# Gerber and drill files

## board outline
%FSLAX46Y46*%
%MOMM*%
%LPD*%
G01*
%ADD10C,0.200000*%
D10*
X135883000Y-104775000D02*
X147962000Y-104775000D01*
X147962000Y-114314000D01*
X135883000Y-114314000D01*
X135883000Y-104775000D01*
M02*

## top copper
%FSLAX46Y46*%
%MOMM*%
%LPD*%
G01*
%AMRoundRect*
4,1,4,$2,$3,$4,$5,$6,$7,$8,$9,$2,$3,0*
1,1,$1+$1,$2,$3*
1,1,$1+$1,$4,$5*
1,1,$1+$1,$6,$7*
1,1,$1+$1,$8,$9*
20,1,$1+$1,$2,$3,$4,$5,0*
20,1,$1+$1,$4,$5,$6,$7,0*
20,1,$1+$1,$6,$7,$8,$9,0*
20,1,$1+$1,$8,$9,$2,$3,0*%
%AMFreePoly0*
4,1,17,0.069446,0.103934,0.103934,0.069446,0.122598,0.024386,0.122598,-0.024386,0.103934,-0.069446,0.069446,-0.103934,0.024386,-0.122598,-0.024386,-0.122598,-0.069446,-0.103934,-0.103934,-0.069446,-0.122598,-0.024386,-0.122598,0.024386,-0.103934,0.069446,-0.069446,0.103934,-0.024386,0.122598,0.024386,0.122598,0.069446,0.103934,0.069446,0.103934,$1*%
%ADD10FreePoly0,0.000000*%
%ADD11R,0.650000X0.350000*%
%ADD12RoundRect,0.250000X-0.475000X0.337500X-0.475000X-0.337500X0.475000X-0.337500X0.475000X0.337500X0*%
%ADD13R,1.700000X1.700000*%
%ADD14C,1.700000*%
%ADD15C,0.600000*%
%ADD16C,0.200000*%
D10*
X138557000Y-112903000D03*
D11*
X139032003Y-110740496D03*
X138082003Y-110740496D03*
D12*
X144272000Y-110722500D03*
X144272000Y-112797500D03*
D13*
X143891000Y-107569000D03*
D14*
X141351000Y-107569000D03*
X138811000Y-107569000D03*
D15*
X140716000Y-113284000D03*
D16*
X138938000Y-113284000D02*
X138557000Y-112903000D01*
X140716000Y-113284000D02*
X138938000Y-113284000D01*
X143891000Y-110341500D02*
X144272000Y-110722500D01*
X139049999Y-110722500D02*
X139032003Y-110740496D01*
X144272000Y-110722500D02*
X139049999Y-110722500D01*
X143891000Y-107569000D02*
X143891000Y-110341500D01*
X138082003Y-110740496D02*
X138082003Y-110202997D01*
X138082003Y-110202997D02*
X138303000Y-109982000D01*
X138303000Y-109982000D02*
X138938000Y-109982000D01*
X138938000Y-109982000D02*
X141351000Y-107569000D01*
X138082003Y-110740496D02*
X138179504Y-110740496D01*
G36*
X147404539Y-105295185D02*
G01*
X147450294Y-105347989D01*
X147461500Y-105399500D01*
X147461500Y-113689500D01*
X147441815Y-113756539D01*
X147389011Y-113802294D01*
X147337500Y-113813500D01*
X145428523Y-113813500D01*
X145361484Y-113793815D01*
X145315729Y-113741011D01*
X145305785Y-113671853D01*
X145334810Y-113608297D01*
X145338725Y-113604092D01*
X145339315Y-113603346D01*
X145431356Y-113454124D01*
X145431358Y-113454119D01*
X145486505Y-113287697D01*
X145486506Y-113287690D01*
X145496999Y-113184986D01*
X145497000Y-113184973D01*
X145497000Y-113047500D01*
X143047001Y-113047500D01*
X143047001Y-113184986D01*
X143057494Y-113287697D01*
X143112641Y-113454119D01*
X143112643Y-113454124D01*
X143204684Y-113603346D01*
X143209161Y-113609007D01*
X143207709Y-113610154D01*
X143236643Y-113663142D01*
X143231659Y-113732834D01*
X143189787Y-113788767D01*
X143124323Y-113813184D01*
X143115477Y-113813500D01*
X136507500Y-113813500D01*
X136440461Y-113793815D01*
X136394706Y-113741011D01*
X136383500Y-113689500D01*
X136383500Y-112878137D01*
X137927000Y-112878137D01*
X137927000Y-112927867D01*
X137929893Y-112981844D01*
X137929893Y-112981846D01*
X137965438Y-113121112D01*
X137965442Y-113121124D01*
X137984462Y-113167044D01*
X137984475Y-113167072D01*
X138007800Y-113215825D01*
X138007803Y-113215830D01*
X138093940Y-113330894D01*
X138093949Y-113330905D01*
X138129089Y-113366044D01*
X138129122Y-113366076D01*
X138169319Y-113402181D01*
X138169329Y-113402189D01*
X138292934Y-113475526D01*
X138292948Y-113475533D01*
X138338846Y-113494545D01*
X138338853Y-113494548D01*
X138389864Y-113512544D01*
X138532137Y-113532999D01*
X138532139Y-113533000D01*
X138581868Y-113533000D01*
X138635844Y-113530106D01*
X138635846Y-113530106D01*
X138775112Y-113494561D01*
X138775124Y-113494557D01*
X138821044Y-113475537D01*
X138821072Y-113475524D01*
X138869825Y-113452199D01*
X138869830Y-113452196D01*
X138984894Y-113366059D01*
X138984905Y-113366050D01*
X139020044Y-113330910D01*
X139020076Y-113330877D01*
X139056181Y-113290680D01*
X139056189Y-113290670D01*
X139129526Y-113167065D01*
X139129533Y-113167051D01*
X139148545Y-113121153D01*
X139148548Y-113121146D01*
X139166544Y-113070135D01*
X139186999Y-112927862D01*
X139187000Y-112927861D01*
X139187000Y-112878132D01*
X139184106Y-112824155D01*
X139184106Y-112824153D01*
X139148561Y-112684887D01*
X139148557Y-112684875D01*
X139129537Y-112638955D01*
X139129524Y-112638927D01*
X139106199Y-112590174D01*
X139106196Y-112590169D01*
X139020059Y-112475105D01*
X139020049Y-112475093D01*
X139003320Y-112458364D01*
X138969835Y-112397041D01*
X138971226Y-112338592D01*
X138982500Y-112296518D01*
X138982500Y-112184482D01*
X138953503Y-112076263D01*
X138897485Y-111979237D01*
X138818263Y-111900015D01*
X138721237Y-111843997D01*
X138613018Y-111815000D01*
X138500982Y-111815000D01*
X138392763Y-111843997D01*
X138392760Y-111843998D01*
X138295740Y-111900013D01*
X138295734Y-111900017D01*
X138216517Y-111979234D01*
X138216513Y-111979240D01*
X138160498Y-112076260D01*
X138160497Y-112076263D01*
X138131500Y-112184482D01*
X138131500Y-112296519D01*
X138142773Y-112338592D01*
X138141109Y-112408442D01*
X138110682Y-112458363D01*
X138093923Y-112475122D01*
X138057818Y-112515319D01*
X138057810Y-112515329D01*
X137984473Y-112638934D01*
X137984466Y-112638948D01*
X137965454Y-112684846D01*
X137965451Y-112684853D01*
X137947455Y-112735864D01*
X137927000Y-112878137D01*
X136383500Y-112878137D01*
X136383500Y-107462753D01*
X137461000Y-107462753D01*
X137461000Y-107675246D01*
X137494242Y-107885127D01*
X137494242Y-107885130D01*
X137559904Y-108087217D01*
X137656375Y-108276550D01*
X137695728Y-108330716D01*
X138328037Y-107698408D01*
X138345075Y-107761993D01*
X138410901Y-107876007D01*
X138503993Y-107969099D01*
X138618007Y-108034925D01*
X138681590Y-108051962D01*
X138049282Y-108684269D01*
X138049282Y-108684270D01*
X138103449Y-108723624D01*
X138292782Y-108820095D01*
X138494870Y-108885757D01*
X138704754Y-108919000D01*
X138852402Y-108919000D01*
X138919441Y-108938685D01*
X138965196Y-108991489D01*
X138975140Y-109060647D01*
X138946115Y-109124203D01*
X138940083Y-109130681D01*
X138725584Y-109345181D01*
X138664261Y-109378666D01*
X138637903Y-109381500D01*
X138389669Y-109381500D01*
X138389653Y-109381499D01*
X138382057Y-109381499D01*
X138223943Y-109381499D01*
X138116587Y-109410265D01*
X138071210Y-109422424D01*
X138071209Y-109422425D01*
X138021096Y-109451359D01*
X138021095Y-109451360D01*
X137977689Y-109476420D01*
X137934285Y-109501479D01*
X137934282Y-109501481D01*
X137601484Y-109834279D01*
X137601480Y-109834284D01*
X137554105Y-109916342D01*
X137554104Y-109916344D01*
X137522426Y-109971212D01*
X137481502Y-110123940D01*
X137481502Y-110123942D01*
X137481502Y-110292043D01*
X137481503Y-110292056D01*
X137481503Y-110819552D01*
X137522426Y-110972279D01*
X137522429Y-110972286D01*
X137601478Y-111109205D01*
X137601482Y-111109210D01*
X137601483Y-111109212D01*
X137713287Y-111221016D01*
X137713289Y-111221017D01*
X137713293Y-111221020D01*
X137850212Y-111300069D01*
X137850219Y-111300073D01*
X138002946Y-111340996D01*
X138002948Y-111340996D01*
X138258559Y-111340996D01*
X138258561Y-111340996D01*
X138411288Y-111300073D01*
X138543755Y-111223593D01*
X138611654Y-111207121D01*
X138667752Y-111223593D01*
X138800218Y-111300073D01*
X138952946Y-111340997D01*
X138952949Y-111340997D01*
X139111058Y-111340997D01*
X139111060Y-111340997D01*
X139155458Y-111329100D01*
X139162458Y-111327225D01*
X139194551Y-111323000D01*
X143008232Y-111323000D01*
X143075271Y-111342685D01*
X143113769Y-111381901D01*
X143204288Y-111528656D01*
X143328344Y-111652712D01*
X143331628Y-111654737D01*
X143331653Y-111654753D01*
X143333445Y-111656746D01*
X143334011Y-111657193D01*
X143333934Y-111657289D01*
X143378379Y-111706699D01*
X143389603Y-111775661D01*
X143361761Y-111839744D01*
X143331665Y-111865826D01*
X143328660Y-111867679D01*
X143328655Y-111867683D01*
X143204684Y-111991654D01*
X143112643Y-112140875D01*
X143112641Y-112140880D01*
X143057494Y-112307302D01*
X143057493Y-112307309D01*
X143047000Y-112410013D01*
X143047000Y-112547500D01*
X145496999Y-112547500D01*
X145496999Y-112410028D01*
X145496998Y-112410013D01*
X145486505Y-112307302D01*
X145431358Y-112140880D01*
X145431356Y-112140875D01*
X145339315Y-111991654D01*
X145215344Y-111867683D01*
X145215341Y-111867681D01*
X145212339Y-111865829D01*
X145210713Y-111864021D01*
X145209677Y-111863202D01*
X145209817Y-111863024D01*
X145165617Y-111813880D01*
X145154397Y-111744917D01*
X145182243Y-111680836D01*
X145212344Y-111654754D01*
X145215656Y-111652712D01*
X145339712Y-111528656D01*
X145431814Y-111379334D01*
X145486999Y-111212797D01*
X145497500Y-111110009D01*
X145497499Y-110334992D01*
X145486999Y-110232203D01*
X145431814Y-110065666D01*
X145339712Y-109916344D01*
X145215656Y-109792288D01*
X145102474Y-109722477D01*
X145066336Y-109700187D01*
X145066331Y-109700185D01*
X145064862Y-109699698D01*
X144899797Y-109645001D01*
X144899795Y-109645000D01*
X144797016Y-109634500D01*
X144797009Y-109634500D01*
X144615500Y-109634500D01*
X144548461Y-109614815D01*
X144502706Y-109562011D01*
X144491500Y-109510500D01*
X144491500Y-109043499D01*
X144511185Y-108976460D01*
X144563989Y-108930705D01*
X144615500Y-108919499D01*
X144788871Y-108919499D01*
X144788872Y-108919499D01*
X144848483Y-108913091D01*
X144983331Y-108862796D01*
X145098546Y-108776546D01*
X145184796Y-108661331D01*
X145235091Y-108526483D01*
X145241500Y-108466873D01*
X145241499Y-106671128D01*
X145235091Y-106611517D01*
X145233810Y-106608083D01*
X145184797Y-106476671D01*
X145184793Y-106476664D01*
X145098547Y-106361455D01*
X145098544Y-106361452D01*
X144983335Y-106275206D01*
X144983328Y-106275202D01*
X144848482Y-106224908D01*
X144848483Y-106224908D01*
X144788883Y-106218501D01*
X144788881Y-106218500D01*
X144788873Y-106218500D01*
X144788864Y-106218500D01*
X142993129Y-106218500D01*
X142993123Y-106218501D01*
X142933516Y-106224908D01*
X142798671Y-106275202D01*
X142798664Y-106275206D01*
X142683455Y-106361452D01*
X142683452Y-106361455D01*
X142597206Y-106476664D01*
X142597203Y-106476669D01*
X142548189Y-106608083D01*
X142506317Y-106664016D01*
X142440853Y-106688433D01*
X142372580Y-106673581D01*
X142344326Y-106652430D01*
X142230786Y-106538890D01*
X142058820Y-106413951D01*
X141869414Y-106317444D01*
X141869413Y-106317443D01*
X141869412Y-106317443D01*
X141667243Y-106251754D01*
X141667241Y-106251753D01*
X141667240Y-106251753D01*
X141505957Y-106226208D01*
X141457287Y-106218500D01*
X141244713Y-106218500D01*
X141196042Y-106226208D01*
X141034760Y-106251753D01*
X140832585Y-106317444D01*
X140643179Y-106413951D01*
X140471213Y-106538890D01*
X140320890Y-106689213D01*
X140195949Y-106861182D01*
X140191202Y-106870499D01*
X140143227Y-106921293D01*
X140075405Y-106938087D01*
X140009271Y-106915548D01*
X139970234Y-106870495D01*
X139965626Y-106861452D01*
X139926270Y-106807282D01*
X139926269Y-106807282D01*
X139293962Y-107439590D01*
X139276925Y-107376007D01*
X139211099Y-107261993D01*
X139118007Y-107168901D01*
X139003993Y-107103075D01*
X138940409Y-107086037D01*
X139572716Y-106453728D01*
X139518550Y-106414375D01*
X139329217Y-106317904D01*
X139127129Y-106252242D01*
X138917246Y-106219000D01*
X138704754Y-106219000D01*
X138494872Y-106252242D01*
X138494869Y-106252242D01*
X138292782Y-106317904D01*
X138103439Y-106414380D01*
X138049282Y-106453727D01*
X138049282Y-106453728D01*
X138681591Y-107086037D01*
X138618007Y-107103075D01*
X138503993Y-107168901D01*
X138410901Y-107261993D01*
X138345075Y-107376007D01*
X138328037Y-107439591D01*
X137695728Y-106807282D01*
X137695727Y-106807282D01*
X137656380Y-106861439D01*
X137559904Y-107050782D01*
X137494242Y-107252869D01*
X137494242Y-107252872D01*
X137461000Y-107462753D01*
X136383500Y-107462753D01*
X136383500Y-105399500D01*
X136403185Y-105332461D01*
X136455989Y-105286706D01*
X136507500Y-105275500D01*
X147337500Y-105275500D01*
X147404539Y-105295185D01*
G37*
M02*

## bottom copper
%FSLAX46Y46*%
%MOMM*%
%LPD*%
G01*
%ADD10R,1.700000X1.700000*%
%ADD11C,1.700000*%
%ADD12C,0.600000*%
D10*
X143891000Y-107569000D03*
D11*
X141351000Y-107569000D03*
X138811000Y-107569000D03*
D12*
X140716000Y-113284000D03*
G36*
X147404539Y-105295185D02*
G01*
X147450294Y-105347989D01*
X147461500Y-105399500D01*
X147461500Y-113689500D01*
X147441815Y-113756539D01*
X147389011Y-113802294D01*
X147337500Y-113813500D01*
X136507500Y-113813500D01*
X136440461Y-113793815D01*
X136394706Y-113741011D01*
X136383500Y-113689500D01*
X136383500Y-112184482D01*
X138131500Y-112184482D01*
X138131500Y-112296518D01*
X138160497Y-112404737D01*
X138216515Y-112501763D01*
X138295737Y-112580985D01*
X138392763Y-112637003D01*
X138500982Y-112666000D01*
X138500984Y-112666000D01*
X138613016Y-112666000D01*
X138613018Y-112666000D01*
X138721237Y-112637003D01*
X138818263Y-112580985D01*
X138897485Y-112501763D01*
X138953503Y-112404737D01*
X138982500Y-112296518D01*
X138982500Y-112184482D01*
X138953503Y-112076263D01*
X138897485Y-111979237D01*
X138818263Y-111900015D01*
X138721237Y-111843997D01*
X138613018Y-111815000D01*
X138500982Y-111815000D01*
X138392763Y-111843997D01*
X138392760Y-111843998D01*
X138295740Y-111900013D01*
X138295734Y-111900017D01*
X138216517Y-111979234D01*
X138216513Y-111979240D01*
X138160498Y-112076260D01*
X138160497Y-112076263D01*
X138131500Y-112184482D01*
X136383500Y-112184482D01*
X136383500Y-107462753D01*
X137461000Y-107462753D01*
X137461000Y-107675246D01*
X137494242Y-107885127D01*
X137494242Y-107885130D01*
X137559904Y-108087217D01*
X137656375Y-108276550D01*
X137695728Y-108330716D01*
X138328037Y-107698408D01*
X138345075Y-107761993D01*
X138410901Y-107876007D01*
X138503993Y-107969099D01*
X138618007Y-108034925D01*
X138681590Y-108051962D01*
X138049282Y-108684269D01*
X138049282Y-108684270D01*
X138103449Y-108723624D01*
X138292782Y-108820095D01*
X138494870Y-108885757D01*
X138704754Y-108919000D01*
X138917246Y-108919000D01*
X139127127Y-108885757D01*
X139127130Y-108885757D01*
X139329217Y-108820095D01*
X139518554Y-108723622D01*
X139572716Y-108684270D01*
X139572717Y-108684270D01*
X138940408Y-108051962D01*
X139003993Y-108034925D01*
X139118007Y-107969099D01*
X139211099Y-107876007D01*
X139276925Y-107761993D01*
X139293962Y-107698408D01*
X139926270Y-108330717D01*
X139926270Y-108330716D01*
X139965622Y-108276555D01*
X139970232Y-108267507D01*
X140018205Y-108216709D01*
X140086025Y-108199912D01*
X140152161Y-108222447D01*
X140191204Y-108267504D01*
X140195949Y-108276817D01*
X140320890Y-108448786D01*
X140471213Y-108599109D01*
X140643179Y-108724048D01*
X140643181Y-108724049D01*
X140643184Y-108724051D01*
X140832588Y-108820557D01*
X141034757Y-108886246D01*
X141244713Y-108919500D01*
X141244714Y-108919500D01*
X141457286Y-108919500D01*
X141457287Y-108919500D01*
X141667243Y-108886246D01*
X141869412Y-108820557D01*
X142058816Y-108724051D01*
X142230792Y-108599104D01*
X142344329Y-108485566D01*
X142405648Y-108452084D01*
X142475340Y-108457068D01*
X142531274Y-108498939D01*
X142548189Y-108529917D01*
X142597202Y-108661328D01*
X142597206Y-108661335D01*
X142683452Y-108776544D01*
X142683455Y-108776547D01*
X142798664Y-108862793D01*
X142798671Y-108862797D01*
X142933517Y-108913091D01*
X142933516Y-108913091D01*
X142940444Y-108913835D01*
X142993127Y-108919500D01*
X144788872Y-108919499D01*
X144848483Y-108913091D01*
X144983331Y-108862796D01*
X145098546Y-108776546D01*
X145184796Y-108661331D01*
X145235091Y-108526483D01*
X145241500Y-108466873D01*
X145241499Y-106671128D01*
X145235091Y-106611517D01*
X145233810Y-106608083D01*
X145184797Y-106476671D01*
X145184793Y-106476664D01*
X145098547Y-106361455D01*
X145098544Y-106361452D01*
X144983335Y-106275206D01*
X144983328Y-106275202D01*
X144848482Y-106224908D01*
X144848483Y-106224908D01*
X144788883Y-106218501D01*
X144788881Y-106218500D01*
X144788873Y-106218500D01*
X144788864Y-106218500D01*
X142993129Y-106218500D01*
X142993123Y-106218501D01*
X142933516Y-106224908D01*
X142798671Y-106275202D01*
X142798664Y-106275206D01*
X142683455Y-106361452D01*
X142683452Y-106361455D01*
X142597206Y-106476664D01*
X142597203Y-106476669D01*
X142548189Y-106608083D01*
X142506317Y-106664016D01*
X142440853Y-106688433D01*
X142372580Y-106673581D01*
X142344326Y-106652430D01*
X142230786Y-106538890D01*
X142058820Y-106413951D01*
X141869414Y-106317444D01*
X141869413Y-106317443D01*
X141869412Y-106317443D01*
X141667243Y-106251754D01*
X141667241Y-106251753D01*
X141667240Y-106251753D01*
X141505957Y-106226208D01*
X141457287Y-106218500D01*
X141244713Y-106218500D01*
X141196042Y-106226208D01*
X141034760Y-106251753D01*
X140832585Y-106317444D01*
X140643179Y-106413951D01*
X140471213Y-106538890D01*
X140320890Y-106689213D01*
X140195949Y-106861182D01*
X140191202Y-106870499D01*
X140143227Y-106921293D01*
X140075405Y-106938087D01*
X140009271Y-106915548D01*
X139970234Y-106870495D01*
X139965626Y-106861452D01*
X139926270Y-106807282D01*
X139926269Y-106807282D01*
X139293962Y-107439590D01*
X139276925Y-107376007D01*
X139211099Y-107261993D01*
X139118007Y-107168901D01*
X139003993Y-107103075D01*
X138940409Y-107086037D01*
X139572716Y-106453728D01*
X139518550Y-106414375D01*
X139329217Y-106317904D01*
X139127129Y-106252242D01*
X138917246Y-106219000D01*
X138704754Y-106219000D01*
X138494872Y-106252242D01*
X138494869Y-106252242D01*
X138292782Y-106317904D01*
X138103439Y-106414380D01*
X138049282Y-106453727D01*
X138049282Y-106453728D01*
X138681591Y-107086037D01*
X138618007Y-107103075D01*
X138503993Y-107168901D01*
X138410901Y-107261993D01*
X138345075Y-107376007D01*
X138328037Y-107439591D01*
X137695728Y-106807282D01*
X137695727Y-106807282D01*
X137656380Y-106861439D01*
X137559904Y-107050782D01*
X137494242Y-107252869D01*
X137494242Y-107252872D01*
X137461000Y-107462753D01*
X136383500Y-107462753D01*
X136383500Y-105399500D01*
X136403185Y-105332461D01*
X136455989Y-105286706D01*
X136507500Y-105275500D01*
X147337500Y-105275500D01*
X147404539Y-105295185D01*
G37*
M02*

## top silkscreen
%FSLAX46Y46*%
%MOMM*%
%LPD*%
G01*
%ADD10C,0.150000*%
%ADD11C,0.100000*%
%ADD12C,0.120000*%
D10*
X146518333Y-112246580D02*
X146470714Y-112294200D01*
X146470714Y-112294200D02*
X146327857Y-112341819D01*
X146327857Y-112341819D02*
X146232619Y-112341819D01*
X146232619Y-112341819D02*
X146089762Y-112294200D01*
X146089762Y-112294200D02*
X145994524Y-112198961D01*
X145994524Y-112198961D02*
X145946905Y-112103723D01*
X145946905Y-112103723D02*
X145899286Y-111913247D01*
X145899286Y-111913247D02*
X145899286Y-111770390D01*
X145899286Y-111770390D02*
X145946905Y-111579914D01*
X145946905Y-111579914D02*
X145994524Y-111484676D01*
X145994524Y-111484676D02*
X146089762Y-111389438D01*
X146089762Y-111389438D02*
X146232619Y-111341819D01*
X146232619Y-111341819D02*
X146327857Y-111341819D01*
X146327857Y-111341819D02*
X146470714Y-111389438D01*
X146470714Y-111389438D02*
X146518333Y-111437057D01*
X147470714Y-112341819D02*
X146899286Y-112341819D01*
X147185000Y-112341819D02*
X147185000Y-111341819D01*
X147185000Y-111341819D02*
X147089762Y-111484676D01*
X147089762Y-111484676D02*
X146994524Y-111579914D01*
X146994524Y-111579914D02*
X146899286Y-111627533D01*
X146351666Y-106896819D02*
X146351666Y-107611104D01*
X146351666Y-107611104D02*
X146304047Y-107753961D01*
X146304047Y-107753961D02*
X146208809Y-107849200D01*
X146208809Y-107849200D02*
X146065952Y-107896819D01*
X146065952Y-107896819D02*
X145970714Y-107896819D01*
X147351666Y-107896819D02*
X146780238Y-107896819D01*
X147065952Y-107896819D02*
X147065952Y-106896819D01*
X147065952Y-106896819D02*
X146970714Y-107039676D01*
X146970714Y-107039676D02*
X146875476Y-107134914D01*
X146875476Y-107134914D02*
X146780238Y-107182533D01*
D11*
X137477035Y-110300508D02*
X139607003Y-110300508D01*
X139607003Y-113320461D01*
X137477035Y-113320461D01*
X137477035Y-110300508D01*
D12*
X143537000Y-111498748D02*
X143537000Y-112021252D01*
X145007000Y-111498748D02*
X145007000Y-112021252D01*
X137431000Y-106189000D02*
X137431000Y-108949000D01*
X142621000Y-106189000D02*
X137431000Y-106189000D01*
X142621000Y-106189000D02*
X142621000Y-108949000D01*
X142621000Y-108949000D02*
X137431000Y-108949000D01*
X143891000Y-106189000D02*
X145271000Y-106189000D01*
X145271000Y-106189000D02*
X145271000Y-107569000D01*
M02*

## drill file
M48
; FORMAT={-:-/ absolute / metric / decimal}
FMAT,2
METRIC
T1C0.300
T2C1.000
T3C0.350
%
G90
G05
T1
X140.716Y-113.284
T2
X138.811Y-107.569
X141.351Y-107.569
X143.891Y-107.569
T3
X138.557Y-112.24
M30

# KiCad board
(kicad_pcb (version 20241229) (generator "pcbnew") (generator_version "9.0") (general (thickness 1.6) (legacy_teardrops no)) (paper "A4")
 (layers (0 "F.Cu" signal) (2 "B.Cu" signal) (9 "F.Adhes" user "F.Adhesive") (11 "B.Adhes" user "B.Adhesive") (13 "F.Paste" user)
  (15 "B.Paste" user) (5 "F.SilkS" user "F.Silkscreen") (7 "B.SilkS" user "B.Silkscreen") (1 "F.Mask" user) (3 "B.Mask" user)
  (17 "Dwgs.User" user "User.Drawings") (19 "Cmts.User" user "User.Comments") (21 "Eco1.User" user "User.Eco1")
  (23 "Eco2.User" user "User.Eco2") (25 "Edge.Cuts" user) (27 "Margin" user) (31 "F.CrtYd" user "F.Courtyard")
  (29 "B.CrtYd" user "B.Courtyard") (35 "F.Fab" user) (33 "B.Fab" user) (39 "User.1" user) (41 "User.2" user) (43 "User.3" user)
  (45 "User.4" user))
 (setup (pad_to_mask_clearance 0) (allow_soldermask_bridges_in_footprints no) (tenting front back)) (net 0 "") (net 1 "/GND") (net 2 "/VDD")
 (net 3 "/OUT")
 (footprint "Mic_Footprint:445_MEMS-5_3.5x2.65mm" (layer "F.Cu") (at 138.557003 112.290496)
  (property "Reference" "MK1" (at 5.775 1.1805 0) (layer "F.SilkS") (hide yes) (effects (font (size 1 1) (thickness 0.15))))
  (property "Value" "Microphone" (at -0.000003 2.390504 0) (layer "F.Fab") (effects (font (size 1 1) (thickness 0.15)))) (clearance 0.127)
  (fp_rect (start -1.079968 -1.989988) (end 1.05 1.029965) (stroke (width 0.1) (type default)) (fill no) (layer "F.SilkS"))
  (pad "" np_thru_hole circle (at -0.000003 -0.049996) (size 0.35 0.35) (drill 0.35) (layers "*.Cu" "*.Mask"))
  (pad "1" smd custom (at -0.000003 0.612504) (size 0.25 0.25) (layers "F.Cu" "F.Mask") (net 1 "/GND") (zone_connect 0)
   (options (clearance outline) (anchor circle)) (primitives))
  (pad "2" smd rect (at 0.475 -1.55) (size 0.65 0.35) (layers "F.Cu" "F.Mask" "F.Paste") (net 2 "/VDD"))
  (pad "3" smd rect (at -0.475 -1.55) (size 0.65 0.35) (layers "F.Cu" "F.Mask" "F.Paste") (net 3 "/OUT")))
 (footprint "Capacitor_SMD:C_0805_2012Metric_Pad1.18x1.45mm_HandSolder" (layer "F.Cu") (at 144.272 111.76 -90)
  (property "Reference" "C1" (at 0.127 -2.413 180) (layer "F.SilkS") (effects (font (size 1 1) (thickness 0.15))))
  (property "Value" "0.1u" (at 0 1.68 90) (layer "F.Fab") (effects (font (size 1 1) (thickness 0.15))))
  (fp_line (start -0.261252 0.735) (end 0.261252 0.735) (stroke (width 0.12) (type solid)) (layer "F.SilkS"))
  (fp_line (start -0.261252 -0.735) (end 0.261252 -0.735) (stroke (width 0.12) (type solid)) (layer "F.SilkS"))
  (pad "1" smd roundrect (at -1.0375 0 270) (size 1.175 1.45) (layers "F.Cu" "F.Mask" "F.Paste") (roundrect_rratio 0.212766) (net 2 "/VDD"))
  (pad "2" smd roundrect (at 1.0375 0 270) (size 1.175 1.45) (layers "F.Cu" "F.Mask" "F.Paste") (roundrect_rratio 0.212766) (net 1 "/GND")))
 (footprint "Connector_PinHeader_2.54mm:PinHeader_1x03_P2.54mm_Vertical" (layer "F.Cu") (at 143.891 107.569 -90)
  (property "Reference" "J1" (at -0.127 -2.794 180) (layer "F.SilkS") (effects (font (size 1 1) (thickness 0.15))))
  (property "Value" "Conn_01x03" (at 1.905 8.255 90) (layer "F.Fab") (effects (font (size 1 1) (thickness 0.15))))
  (fp_line (start -1.38 6.46) (end 1.38 6.46) (stroke (width 0.12) (type solid)) (layer "F.SilkS"))
  (fp_line (start -1.38 1.27) (end -1.38 6.46) (stroke (width 0.12) (type solid)) (layer "F.SilkS"))
  (fp_line (start -1.38 1.27) (end 1.38 1.27) (stroke (width 0.12) (type solid)) (layer "F.SilkS"))
  (fp_line (start 1.38 1.27) (end 1.38 6.46) (stroke (width 0.12) (type solid)) (layer "F.SilkS"))
  (fp_line (start -1.38 0) (end -1.38 -1.38) (stroke (width 0.12) (type solid)) (layer "F.SilkS"))
  (fp_line (start -1.38 -1.38) (end 0 -1.38) (stroke (width 0.12) (type solid)) (layer "F.SilkS"))
  (pad "1" thru_hole rect (at 0 0 270) (size 1.7 1.7) (drill 1) (layers "*.Cu" "*.Mask") (remove_unused_layers no) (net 2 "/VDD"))
  (pad "2" thru_hole circle (at 0 2.54 270) (size 1.7 1.7) (drill 1) (layers "*.Cu" "*.Mask") (remove_unused_layers no) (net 3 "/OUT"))
  (pad "3" thru_hole circle (at 0 5.08 270) (size 1.7 1.7) (drill 1) (layers "*.Cu" "*.Mask") (remove_unused_layers no) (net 1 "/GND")))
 (gr_rect (start 135.883 104.775) (end 147.962 114.314) (stroke (width 0.2) (type solid)) (fill no) (layer "Edge.Cuts"))
 (segment (start 138.938 113.284) (end 138.557 112.903) (width 0.2) (layer "F.Cu") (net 1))
 (segment (start 140.716 113.284) (end 138.938 113.284) (width 0.2) (layer "F.Cu") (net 1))
 (via (at 140.716 113.284) (size 0.6) (drill 0.3) (layers "F.Cu" "B.Cu") (free yes) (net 1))
 (segment (start 143.891 110.3415) (end 144.272 110.7225) (width 0.2) (layer "F.Cu") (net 2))
 (segment (start 139.049999 110.7225) (end 139.032003 110.740496) (width 0.2) (layer "F.Cu") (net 2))
 (segment (start 144.272 110.7225) (end 139.049999 110.7225) (width 0.2) (layer "F.Cu") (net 2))
 (segment (start 143.891 107.569) (end 143.891 110.3415) (width 0.2) (layer "F.Cu") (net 2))
 (segment (start 138.082003 110.740496) (end 138.082003 110.202997) (width 0.2) (layer "F.Cu") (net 3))
 (segment (start 138.082003 110.202997) (end 138.303 109.982) (width 0.2) (layer "F.Cu") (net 3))
 (segment (start 138.303 109.982) (end 138.938 109.982) (width 0.2) (layer "F.Cu") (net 3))
 (segment (start 138.938 109.982) (end 141.351 107.569) (width 0.2) (layer "F.Cu") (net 3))
 (segment (start 138.082003 110.740496) (end 138.179504 110.740496) (width 0.2) (layer "F.Cu") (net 3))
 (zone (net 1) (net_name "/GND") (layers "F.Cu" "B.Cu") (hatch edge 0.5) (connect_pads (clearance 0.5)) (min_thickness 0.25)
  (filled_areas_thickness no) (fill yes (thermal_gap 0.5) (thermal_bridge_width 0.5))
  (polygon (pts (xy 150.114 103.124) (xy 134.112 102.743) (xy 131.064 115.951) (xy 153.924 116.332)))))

